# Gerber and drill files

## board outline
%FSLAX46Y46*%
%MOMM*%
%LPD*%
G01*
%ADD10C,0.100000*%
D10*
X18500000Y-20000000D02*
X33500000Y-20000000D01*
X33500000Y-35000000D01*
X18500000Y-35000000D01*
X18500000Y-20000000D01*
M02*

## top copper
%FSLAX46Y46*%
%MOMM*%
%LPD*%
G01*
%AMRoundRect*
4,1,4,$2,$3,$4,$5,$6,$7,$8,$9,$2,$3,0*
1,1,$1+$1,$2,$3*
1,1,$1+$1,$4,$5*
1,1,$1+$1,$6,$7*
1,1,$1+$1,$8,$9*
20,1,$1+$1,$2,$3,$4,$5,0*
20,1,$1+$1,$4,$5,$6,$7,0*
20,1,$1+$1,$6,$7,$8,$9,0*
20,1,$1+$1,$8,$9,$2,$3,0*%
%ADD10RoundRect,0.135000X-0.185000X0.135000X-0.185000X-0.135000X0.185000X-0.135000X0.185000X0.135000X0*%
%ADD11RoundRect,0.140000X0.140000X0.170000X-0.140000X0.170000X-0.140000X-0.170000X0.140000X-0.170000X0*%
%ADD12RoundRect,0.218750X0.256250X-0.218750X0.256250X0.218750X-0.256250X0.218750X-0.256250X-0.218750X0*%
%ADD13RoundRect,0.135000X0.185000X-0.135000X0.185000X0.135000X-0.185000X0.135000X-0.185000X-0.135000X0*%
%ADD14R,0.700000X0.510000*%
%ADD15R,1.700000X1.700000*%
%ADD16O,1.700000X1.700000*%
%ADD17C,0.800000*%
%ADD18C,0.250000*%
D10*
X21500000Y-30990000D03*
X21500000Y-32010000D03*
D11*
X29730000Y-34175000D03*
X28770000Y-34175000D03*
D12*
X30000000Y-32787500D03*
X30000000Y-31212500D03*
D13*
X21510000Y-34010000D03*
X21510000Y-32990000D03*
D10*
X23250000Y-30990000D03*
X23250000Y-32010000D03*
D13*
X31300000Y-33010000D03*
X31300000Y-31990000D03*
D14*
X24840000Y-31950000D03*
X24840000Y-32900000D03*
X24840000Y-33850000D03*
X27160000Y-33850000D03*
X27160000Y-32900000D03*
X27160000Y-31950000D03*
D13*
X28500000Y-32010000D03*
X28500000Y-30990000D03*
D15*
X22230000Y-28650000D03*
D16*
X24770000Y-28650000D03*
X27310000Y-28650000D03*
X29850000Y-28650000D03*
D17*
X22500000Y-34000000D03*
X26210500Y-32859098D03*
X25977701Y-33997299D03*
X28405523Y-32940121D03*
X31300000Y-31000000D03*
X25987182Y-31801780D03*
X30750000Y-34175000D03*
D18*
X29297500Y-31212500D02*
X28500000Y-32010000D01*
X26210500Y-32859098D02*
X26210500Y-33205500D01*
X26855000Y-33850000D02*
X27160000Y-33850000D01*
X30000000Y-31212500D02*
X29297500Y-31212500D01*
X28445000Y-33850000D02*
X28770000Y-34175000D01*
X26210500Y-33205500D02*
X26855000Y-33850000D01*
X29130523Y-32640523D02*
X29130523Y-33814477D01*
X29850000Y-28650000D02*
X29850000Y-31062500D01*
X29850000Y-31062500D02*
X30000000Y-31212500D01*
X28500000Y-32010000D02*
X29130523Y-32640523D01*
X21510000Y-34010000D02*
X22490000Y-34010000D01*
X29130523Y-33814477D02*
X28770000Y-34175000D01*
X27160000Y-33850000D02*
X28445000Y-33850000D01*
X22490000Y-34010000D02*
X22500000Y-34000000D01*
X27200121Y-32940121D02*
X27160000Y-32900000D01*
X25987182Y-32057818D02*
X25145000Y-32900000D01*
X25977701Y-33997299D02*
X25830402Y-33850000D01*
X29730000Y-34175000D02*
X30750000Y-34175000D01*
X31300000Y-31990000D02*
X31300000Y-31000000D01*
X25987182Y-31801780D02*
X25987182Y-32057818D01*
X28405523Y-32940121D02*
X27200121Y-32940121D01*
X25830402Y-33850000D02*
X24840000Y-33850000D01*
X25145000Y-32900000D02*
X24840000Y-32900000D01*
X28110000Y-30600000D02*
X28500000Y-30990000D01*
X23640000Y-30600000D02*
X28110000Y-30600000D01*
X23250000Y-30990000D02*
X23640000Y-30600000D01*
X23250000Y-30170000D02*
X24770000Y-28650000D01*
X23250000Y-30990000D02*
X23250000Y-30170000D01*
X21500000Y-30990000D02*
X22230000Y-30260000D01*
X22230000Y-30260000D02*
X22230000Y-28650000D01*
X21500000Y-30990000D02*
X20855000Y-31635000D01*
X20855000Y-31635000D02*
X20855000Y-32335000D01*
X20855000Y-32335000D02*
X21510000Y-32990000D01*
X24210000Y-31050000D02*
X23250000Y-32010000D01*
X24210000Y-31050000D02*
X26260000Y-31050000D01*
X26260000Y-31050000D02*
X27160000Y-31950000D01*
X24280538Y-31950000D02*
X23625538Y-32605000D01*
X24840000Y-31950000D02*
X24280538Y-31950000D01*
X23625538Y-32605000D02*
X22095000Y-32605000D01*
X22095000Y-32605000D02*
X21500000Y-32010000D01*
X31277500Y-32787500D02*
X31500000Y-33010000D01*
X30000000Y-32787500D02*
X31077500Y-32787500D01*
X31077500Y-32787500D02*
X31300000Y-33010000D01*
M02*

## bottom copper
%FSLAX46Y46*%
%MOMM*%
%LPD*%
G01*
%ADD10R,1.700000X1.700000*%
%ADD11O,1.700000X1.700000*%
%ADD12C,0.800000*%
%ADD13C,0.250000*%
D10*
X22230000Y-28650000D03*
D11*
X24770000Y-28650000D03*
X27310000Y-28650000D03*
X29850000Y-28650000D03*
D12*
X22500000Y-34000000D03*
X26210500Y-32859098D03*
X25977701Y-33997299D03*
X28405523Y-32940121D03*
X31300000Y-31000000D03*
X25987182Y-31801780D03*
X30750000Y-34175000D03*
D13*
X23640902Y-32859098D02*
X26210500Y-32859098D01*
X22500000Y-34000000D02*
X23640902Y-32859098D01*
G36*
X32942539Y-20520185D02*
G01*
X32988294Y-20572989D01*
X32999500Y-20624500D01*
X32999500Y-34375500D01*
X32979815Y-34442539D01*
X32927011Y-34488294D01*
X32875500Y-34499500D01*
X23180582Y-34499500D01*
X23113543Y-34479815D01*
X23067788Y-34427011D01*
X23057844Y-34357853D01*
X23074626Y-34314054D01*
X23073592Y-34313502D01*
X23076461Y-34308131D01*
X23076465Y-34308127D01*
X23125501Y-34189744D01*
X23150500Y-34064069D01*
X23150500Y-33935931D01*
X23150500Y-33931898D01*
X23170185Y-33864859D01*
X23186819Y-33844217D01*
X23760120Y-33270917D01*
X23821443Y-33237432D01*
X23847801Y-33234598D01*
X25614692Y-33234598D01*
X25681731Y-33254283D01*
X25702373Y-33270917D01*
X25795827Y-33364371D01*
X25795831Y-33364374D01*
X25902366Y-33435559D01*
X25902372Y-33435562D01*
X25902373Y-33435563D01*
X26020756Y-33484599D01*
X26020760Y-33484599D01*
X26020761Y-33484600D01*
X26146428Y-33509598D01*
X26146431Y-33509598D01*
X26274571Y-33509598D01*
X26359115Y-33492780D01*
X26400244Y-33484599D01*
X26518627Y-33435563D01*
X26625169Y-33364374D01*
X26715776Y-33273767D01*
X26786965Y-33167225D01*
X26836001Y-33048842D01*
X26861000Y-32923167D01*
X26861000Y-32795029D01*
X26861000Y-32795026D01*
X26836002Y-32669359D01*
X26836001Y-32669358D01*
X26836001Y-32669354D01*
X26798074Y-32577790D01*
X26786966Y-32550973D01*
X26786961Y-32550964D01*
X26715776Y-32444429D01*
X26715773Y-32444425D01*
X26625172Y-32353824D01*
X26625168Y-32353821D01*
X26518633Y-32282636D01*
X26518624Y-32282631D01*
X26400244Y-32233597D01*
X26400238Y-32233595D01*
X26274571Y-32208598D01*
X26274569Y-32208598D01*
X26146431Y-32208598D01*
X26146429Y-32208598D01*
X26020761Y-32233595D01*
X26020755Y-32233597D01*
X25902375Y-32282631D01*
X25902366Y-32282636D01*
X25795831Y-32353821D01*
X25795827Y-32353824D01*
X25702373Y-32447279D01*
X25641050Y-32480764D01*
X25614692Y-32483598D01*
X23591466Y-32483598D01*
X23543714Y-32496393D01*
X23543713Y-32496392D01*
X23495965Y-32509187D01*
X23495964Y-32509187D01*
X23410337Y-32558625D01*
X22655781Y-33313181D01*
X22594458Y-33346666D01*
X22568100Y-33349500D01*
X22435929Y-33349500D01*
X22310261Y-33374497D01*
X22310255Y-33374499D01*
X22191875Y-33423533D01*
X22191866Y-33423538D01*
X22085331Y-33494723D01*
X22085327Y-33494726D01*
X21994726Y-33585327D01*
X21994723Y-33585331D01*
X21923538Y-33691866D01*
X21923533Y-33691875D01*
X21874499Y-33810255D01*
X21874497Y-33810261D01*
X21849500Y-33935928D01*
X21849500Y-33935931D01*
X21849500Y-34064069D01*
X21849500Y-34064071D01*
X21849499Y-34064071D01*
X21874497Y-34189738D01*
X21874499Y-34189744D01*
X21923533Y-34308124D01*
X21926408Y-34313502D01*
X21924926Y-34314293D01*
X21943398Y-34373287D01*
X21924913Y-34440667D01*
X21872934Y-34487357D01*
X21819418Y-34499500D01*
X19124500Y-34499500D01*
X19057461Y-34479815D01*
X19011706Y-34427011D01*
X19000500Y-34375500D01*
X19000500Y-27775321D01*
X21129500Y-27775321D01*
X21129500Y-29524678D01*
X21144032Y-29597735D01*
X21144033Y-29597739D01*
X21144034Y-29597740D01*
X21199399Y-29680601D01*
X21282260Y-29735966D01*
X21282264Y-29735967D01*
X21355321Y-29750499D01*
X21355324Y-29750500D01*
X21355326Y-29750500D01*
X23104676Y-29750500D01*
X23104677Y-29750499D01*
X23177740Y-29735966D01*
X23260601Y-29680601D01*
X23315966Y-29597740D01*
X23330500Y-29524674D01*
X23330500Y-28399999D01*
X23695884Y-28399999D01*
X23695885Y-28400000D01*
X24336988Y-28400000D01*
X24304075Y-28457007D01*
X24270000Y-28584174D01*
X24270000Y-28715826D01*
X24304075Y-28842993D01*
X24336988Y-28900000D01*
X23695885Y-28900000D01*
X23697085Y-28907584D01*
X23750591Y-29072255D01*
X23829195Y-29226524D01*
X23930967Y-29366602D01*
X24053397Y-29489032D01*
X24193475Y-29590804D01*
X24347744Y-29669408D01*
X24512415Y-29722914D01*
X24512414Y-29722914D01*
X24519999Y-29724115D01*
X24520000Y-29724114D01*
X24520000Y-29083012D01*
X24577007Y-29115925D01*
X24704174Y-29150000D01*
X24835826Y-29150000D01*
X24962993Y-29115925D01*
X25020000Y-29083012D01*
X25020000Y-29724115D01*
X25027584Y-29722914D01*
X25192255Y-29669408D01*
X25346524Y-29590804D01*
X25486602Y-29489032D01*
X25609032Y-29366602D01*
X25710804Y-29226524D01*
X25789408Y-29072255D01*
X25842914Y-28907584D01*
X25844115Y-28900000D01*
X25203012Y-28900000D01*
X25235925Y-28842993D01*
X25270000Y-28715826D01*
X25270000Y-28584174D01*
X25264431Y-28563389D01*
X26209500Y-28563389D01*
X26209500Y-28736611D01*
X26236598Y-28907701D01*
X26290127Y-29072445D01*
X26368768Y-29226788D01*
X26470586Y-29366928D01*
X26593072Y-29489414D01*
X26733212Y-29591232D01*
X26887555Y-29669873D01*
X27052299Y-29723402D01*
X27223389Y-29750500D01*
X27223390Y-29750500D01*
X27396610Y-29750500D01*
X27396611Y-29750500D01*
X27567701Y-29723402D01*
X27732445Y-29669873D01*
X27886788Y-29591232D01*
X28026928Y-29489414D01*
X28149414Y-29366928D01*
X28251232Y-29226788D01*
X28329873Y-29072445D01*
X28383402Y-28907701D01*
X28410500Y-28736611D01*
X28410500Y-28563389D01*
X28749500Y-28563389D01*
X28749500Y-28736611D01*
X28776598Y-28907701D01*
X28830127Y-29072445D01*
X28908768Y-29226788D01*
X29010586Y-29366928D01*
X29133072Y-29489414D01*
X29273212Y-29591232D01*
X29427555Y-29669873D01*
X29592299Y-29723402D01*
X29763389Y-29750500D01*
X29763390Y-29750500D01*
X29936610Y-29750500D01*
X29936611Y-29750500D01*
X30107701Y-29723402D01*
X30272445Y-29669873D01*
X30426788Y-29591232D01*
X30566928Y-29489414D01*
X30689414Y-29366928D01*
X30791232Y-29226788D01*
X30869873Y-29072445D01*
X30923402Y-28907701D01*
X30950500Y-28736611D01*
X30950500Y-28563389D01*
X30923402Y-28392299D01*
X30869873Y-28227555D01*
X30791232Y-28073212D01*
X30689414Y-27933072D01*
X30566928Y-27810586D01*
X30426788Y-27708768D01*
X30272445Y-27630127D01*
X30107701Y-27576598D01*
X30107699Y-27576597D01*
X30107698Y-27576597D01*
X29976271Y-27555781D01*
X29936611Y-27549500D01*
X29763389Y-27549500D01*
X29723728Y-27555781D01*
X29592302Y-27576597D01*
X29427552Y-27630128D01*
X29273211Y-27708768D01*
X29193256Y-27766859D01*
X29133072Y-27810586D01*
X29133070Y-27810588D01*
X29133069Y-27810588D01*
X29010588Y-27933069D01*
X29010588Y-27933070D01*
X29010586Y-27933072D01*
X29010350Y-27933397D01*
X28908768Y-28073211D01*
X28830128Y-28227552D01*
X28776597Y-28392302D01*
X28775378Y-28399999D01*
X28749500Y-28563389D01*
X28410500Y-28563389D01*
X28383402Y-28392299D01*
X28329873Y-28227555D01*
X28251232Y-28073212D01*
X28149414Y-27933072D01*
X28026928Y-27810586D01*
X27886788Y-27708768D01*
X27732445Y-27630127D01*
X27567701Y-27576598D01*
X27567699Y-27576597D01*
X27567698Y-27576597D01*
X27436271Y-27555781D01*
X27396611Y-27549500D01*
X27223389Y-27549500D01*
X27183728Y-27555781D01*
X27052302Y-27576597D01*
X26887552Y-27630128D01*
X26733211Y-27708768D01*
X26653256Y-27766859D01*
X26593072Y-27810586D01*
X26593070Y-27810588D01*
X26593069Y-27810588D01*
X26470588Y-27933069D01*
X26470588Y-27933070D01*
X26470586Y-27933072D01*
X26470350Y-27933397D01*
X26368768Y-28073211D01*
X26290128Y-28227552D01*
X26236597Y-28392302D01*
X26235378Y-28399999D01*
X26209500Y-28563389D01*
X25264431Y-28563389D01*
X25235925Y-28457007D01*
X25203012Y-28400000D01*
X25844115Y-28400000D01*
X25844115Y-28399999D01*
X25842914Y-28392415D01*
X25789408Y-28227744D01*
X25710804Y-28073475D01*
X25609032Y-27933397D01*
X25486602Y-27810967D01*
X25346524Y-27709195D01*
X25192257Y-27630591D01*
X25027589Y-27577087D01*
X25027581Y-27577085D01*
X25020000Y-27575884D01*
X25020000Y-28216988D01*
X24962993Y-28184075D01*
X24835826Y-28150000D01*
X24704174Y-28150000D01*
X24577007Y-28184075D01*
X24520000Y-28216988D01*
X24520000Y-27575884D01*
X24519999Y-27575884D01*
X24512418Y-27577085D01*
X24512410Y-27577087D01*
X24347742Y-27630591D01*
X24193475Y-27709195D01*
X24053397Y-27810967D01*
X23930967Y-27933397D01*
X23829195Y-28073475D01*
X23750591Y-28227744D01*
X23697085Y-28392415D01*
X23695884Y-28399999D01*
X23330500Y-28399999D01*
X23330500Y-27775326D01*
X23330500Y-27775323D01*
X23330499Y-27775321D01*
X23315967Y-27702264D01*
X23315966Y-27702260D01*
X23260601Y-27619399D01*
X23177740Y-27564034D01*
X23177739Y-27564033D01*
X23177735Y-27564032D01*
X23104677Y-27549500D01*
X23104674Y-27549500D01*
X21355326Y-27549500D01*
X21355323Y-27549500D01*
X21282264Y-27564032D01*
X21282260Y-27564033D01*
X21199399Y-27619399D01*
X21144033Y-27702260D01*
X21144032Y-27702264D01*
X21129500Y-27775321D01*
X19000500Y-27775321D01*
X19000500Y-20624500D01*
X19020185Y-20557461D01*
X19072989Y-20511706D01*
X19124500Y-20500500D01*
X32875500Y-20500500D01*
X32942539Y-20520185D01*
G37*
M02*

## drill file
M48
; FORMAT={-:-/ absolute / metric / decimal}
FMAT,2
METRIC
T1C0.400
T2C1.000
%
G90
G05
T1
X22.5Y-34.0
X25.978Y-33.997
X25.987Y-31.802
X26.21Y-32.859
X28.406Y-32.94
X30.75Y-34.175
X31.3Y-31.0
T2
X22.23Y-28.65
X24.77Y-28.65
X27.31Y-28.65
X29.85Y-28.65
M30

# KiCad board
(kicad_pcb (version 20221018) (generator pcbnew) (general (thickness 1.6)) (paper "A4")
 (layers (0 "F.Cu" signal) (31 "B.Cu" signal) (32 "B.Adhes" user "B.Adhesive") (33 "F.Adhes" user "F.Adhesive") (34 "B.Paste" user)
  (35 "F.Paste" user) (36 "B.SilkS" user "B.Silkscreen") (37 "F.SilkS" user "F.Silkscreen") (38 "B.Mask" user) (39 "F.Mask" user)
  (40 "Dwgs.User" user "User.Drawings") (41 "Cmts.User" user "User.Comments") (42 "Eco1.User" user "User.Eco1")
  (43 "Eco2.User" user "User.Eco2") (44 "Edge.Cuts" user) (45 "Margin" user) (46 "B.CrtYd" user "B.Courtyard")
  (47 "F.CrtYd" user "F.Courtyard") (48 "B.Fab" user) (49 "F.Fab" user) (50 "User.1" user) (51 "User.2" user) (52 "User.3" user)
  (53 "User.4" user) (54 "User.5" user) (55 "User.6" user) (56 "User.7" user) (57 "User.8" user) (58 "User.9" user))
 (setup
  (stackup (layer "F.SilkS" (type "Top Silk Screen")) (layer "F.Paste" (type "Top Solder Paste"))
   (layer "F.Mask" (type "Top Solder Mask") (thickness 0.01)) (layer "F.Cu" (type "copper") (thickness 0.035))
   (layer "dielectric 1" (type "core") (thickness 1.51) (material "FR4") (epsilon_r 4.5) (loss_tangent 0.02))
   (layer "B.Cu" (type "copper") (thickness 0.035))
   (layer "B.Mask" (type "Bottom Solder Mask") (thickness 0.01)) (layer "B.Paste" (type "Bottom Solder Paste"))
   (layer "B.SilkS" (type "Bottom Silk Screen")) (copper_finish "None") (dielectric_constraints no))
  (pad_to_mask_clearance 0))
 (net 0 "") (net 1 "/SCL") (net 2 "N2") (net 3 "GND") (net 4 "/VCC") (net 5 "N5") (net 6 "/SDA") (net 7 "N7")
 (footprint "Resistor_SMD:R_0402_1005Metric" (layer "F.Cu") (at 21.5 31.5 -90)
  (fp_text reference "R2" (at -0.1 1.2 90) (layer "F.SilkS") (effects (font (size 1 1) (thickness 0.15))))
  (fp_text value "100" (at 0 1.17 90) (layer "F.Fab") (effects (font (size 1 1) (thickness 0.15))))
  (pad "1" smd roundrect (at -0.51 0 270) (size 0.54 0.64) (layers "F.Cu" "F.Paste" "F.Mask") (roundrect_rratio 0.25) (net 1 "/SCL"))
  (pad "2" smd roundrect (at 0.51 0 270) (size 0.54 0.64) (layers "F.Cu" "F.Paste" "F.Mask") (roundrect_rratio 0.25) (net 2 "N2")))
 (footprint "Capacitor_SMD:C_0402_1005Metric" (layer "F.Cu") (at 29.25 34.175 180)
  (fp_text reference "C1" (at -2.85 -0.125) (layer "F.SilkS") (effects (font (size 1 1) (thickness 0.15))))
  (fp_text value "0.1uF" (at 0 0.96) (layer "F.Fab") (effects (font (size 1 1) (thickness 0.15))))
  (pad "1" smd roundrect (at -0.48 0 180) (size 0.56 0.62) (layers "F.Cu" "F.Paste" "F.Mask") (roundrect_rratio 0.25) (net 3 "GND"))
  (pad "2" smd roundrect (at 0.48 0 180) (size 0.56 0.62) (layers "F.Cu" "F.Paste" "F.Mask") (roundrect_rratio 0.25) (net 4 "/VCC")))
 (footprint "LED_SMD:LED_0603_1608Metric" (layer "F.Cu") (at 30 32 90)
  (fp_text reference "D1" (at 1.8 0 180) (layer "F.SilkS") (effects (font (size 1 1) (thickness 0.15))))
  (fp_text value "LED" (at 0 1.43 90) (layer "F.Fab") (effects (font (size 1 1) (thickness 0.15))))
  (pad "1" smd roundrect (at -0.7875 0 90) (size 0.875 0.95) (layers "F.Cu" "F.Paste" "F.Mask") (roundrect_rratio 0.25) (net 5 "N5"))
  (pad "2" smd roundrect (at 0.7875 0 90) (size 0.875 0.95) (layers "F.Cu" "F.Paste" "F.Mask") (roundrect_rratio 0.25) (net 4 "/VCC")))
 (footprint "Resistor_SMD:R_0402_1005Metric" (layer "F.Cu") (at 21.51 33.5 90)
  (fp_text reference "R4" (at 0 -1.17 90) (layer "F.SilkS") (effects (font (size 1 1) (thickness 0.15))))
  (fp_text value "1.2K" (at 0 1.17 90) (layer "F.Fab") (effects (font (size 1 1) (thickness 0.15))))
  (pad "1" smd roundrect (at -0.51 0 90) (size 0.54 0.64) (layers "F.Cu" "F.Paste" "F.Mask") (roundrect_rratio 0.25) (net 4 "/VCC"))
  (pad "2" smd roundrect (at 0.51 0 90) (size 0.54 0.64) (layers "F.Cu" "F.Paste" "F.Mask") (roundrect_rratio 0.25) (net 1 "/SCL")))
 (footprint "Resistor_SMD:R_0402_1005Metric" (layer "F.Cu") (at 23.25 31.5 -90)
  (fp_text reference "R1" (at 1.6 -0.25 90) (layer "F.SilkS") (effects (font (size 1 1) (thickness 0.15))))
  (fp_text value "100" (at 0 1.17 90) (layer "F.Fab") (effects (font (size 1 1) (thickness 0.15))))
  (pad "1" smd roundrect (at -0.51 0 270) (size 0.54 0.64) (layers "F.Cu" "F.Paste" "F.Mask") (roundrect_rratio 0.25) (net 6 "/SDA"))
  (pad "2" smd roundrect (at 0.51 0 270) (size 0.54 0.64) (layers "F.Cu" "F.Paste" "F.Mask") (roundrect_rratio 0.25) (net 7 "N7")))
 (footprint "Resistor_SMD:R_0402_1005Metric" (layer "F.Cu") (at 31.3 32.5 90)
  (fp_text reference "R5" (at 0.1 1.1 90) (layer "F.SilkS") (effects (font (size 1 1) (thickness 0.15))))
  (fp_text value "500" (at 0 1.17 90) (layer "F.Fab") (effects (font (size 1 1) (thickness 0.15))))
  (pad "1" smd roundrect (at -0.51 0 90) (size 0.54 0.64) (layers "F.Cu" "F.Paste" "F.Mask") (roundrect_rratio 0.25) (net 5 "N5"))
  (pad "2" smd roundrect (at 0.51 0 90) (size 0.54 0.64) (layers "F.Cu" "F.Paste" "F.Mask") (roundrect_rratio 0.25) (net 3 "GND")))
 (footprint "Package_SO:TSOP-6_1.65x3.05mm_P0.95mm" (layer "F.Cu") (at 26 32.9)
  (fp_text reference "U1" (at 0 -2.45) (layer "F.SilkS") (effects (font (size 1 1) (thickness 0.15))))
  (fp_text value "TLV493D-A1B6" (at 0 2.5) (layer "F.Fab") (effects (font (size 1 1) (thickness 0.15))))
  (pad "1" smd rect (at -1.16 -0.95) (size 0.7 0.51) (layers "F.Cu" "F.Paste" "F.Mask") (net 2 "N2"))
  (pad "2" smd rect (at -1.16 0) (size 0.7 0.51) (layers "F.Cu" "F.Paste" "F.Mask") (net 3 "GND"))
  (pad "3" smd rect (at -1.16 0.95) (size 0.7 0.51) (layers "F.Cu" "F.Paste" "F.Mask") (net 3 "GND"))
  (pad "4" smd rect (at 1.16 0.95) (size 0.7 0.51) (layers "F.Cu" "F.Paste" "F.Mask") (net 4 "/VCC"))
  (pad "5" smd rect (at 1.16 0) (size 0.7 0.51) (layers "F.Cu" "F.Paste" "F.Mask") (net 3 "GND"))
  (pad "6" smd rect (at 1.16 -0.95) (size 0.7 0.51) (layers "F.Cu" "F.Paste" "F.Mask") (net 7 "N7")))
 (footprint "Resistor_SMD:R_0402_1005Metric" (layer "F.Cu") (at 28.5 31.5 90)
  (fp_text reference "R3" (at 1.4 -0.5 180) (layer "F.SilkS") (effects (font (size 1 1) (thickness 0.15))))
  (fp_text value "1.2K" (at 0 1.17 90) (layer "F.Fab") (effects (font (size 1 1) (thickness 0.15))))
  (pad "1" smd roundrect (at -0.51 0 90) (size 0.54 0.64) (layers "F.Cu" "F.Paste" "F.Mask") (roundrect_rratio 0.25) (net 4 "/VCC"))
  (pad "2" smd roundrect (at 0.51 0 90) (size 0.54 0.64) (layers "F.Cu" "F.Paste" "F.Mask") (roundrect_rratio 0.25) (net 6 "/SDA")))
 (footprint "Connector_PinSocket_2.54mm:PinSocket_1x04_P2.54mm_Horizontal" (layer "B.Cu") (at 22.23 28.65 -90)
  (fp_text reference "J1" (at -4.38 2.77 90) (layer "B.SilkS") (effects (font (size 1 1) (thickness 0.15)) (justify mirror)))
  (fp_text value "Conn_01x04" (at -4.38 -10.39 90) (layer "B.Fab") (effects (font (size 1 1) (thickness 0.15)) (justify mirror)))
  (pad "1" thru_hole rect (at 0 0 270) (size 1.7 1.7) (drill 1) (layers "*.Cu" "*.Mask") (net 4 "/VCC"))
  (pad "2" thru_hole oval (at 0 -2.54 270) (size 1.7 1.7) (drill 1) (layers "*.Cu" "*.Mask") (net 3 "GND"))
  (pad "3" thru_hole oval (at 0 -5.08 270) (size 1.7 1.7) (drill 1) (layers "*.Cu" "*.Mask") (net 6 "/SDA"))
  (pad "4" thru_hole oval (at 0 -7.62 270) (size 1.7 1.7) (drill 1) (layers "*.Cu" "*.Mask") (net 1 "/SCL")))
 (gr_rect (start 18.5 20) (end 33.5 35) (stroke (width 0.1) (type default)) (fill none) (layer "Edge.Cuts"))
 (segment (start 29.2975 31.2125) (end 28.5 32.01) (width 0.25) (layer "F.Cu") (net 4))
 (segment (start 26.2105 32.859098) (end 26.2105 33.2055) (width 0.25) (layer "F.Cu") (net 4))
 (segment (start 26.855 33.85) (end 27.16 33.85) (width 0.25) (layer "F.Cu") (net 4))
 (segment (start 30 31.2125) (end 29.2975 31.2125) (width 0.25) (layer "F.Cu") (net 4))
 (segment (start 28.445 33.85) (end 28.77 34.175) (width 0.25) (layer "F.Cu") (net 4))
 (segment (start 26.2105 33.2055) (end 26.855 33.85) (width 0.25) (layer "F.Cu") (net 4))
 (segment (start 29.130523 32.640523) (end 29.130523 33.814477) (width 0.25) (layer "F.Cu") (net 4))
 (segment (start 29.85 28.65) (end 29.85 31.0625) (width 0.25) (layer "F.Cu") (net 4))
 (segment (start 29.85 31.0625) (end 30 31.2125) (width 0.25) (layer "F.Cu") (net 4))
 (segment (start 28.5 32.01) (end 29.130523 32.640523) (width 0.25) (layer "F.Cu") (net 4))
 (segment (start 21.51 34.01) (end 22.49 34.01) (width 0.25) (layer "F.Cu") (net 4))
 (segment (start 29.130523 33.814477) (end 28.77 34.175) (width 0.25) (layer "F.Cu") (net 4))
 (segment (start 27.16 33.85) (end 28.445 33.85) (width 0.25) (layer "F.Cu") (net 4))
 (segment (start 22.49 34.01) (end 22.5 34) (width 0.25) (layer "F.Cu") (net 4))
 (via (at 22.5 34) (size 0.8) (drill 0.4) (layers "F.Cu" "B.Cu") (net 4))
 (via (at 26.2105 32.859098) (size 0.8) (drill 0.4) (layers "F.Cu" "B.Cu") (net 4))
 (segment (start 23.640902 32.859098) (end 26.2105 32.859098) (width 0.25) (layer "B.Cu") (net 4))
 (segment (start 22.5 34) (end 23.640902 32.859098) (width 0.25) (layer "B.Cu") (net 4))
 (segment (start 27.200121 32.940121) (end 27.16 32.9) (width 0.25) (layer "F.Cu") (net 3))
 (segment (start 25.987182 32.057818) (end 25.145 32.9) (width 0.25) (layer "F.Cu") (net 3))
 (segment (start 25.977701 33.997299) (end 25.830402 33.85) (width 0.25) (layer "F.Cu") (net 3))
 (segment (start 29.73 34.175) (end 30.75 34.175) (width 0.25) (layer "F.Cu") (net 3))
 (segment (start 31.3 31.99) (end 31.3 31) (width 0.25) (layer "F.Cu") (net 3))
 (segment (start 25.987182 31.80178) (end 25.987182 32.057818) (width 0.25) (layer "F.Cu") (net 3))
 (segment (start 28.405523 32.940121) (end 27.200121 32.940121) (width 0.25) (layer "F.Cu") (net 3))
 (segment (start 25.830402 33.85) (end 24.84 33.85) (width 0.25) (layer "F.Cu") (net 3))
 (segment (start 25.145 32.9) (end 24.84 32.9) (width 0.25) (layer "F.Cu") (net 3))
 (via (at 25.977701 33.997299) (size 0.8) (drill 0.4) (layers "F.Cu" "B.Cu") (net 3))
 (via (at 28.405523 32.940121) (size 0.8) (drill 0.4) (layers "F.Cu" "B.Cu") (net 3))
 (via (at 31.3 31) (size 0.8) (drill 0.4) (layers "F.Cu" "B.Cu") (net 3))
 (via (at 25.987182 31.80178) (size 0.8) (drill 0.4) (layers "F.Cu" "B.Cu") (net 3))
 (via (at 30.75 34.175) (size 0.8) (drill 0.4) (layers "F.Cu" "B.Cu") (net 3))
 (segment (start 28.11 30.6) (end 28.5 30.99) (width 0.25) (layer "F.Cu") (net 6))
 (segment (start 23.64 30.6) (end 28.11 30.6) (width 0.25) (layer "F.Cu") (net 6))
 (segment (start 23.25 30.99) (end 23.64 30.6) (width 0.25) (layer "F.Cu") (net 6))
 (segment (start 23.25 30.17) (end 24.77 28.65) (width 0.25) (layer "F.Cu") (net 6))
 (segment (start 23.25 30.99) (end 23.25 30.17) (width 0.25) (layer "F.Cu") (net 6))
 (segment (start 21.5 30.99) (end 22.23 30.26) (width 0.25) (layer "F.Cu") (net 1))
 (segment (start 22.23 30.26) (end 22.23 28.65) (width 0.25) (layer "F.Cu") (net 1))
 (segment (start 21.5 30.99) (end 20.855 31.635) (width 0.25) (layer "F.Cu") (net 1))
 (segment (start 20.855 31.635) (end 20.855 32.335) (width 0.25) (layer "F.Cu") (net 1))
 (segment (start 20.855 32.335) (end 21.51 32.99) (width 0.25) (layer "F.Cu") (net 1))
 (segment (start 24.21 31.05) (end 23.25 32.01) (width 0.25) (layer "F.Cu") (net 7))
 (segment (start 24.21 31.05) (end 26.26 31.05) (width 0.25) (layer "F.Cu") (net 7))
 (segment (start 26.26 31.05) (end 27.16 31.95) (width 0.25) (layer "F.Cu") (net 7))
 (segment (start 24.280538 31.95) (end 23.625538 32.605) (width 0.25) (layer "F.Cu") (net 2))
 (segment (start 24.84 31.95) (end 24.280538 31.95) (width 0.25) (layer "F.Cu") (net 2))
 (segment (start 23.625538 32.605) (end 22.095 32.605) (width 0.25) (layer "F.Cu") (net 2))
 (segment (start 22.095 32.605) (end 21.5 32.01) (width 0.25) (layer "F.Cu") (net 2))
 (segment (start 31.2775 32.7875) (end 31.5 33.01) (width 0.25) (layer "F.Cu") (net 5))
 (segment (start 30 32.7875) (end 31.0775 32.7875) (width 0.25) (layer "F.Cu") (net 5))
 (segment (start 31.0775 32.7875) (end 31.3 33.01) (width 0.25) (layer "F.Cu") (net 5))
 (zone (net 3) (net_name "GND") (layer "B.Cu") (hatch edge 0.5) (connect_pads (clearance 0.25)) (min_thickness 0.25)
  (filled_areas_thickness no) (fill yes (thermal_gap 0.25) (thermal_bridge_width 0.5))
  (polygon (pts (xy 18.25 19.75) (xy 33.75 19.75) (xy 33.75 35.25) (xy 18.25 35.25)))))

